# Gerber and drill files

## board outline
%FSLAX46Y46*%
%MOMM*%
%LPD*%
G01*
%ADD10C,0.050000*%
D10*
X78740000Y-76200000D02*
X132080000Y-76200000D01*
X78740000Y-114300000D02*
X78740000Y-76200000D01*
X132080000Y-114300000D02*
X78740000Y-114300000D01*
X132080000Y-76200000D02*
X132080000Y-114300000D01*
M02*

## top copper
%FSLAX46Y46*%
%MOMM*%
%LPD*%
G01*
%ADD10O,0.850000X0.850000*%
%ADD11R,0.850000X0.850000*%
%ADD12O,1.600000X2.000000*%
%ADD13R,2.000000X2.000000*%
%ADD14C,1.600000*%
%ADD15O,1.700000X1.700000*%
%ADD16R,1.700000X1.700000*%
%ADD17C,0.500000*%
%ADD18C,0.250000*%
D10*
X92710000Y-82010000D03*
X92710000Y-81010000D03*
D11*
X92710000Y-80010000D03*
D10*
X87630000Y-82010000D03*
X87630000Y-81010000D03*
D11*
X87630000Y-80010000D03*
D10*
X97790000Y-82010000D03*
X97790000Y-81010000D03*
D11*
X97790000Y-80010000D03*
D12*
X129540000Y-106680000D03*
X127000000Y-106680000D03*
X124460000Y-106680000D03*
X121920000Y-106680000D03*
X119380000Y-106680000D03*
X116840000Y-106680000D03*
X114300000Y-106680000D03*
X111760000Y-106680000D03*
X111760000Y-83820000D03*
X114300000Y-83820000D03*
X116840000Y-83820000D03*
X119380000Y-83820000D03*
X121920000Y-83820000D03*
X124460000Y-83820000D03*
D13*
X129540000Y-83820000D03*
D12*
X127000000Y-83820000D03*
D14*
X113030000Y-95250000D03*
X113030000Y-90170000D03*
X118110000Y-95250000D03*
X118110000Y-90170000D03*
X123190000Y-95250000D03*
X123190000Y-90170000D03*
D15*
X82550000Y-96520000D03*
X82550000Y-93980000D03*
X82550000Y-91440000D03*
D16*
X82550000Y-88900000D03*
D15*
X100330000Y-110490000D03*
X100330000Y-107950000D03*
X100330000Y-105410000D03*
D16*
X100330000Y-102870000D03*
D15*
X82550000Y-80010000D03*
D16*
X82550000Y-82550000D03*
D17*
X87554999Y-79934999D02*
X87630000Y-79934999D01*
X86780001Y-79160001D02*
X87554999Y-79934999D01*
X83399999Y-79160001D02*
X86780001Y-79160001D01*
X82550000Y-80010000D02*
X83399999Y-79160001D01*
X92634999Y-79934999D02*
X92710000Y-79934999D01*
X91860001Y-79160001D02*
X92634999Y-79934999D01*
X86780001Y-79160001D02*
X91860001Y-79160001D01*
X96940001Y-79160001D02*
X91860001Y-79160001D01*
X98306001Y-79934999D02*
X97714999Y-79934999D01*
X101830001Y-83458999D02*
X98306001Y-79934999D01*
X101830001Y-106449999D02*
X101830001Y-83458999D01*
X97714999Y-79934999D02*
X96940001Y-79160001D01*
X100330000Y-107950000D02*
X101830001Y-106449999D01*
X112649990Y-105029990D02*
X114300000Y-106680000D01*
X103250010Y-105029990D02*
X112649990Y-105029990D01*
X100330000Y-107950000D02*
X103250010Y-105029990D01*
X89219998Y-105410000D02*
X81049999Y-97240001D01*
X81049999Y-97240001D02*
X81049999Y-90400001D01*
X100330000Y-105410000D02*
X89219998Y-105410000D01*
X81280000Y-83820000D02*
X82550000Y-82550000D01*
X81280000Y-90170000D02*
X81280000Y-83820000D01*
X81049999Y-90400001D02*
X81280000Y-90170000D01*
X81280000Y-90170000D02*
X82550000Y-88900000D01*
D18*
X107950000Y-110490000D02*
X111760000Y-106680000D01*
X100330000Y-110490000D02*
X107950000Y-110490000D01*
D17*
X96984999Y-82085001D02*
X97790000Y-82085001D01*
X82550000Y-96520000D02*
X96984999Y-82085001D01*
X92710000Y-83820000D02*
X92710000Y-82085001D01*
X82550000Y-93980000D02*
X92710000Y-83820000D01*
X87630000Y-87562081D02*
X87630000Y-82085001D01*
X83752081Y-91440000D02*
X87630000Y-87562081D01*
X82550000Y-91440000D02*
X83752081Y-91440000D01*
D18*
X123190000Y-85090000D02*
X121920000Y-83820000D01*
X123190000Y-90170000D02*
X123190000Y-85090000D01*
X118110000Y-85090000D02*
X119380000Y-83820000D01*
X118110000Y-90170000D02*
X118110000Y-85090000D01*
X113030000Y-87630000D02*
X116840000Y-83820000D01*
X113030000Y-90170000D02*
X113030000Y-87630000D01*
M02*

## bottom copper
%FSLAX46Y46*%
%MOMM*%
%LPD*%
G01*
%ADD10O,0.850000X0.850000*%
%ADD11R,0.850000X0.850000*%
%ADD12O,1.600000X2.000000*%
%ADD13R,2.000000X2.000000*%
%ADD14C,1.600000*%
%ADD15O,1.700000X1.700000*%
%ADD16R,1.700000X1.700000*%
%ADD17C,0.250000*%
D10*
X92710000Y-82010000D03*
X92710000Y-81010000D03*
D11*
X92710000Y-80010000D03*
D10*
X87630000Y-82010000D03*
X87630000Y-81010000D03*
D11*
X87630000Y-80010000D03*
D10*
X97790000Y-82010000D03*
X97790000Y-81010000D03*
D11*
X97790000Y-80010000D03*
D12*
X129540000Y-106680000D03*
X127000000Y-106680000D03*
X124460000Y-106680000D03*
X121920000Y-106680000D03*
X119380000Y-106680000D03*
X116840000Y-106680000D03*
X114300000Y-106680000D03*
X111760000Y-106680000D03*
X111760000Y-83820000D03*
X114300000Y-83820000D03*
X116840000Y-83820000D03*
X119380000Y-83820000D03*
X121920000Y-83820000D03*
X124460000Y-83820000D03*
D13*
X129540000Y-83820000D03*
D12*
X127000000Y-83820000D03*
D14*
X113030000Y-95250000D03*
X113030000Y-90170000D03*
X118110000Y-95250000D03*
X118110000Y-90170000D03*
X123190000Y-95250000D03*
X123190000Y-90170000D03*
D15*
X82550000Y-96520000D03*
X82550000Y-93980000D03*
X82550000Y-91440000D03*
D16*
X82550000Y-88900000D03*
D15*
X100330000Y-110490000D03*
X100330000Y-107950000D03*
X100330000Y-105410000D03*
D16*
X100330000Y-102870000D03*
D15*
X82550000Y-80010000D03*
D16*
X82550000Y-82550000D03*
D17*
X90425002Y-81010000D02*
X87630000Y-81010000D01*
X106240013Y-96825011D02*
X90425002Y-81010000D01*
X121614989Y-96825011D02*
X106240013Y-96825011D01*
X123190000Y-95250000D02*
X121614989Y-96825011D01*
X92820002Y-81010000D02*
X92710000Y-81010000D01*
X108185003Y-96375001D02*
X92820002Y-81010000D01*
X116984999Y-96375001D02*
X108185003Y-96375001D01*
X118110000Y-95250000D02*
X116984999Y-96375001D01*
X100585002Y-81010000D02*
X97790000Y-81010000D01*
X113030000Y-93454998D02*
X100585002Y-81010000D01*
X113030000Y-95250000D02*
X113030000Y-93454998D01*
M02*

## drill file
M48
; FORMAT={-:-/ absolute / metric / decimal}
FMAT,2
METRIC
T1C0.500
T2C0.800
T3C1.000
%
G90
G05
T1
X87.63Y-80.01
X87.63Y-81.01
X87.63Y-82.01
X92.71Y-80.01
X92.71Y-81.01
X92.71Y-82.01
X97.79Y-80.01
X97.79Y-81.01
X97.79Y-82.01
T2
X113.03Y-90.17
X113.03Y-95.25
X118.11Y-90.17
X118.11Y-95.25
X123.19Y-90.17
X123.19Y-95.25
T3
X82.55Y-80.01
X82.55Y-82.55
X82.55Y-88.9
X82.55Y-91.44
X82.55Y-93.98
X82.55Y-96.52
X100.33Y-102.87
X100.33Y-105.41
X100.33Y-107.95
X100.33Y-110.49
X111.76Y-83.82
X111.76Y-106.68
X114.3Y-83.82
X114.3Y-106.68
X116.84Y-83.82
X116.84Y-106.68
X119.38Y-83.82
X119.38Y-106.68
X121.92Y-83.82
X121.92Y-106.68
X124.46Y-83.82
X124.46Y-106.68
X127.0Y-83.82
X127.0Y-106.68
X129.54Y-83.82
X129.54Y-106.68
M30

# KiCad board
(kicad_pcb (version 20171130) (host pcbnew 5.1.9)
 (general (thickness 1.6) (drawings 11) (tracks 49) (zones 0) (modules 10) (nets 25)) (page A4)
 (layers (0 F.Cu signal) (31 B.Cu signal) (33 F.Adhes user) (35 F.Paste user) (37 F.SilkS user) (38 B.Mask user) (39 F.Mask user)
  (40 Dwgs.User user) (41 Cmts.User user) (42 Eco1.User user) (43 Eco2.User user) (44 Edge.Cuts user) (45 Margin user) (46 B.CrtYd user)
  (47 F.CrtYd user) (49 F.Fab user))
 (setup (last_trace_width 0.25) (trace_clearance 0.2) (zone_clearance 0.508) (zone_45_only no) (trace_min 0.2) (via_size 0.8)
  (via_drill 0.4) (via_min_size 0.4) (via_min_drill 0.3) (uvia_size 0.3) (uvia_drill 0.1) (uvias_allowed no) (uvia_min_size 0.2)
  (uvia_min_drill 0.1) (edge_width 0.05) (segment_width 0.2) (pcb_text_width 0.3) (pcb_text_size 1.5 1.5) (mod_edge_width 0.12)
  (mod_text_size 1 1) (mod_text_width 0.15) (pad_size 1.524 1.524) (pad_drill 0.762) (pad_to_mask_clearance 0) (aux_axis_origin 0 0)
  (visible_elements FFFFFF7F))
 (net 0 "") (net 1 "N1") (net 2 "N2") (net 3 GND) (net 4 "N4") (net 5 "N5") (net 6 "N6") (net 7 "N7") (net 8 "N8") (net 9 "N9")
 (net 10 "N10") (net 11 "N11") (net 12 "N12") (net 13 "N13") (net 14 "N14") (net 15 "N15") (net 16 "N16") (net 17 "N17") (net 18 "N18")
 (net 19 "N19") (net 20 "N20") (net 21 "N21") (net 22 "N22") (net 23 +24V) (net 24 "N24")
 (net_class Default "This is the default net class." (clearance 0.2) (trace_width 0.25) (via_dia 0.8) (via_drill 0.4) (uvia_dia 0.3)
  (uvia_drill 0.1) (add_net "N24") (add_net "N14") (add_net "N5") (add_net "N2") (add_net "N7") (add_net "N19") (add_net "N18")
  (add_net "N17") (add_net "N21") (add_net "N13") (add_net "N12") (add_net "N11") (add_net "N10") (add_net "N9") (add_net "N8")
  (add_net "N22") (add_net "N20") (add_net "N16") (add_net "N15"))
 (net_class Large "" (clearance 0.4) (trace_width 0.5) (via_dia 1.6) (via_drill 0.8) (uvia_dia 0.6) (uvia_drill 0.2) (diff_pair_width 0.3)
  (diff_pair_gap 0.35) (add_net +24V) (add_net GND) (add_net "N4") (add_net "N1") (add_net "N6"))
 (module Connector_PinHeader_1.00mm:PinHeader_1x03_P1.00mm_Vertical (layer F.Cu) (at 92.71 80.01)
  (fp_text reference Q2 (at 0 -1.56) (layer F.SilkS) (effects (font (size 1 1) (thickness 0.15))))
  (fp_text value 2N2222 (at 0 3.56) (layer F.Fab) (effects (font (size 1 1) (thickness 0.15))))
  (pad 3 thru_hole oval (at 0 2) (size 0.85 0.85) (drill 0.5) (layers *.Cu *.Mask) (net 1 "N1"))
  (pad 2 thru_hole oval (at 0 1) (size 0.85 0.85) (drill 0.5) (layers *.Cu *.Mask) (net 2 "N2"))
  (pad 1 thru_hole rect (at 0 0) (size 0.85 0.85) (drill 0.5) (layers *.Cu *.Mask) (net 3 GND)))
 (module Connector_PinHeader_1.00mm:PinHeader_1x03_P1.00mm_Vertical (layer F.Cu) (at 87.63 80.01)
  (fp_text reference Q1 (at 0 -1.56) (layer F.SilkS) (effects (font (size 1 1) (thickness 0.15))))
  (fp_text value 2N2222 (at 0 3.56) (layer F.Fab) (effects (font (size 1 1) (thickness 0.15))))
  (pad 3 thru_hole oval (at 0 2) (size 0.85 0.85) (drill 0.5) (layers *.Cu *.Mask) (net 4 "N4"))
  (pad 2 thru_hole oval (at 0 1) (size 0.85 0.85) (drill 0.5) (layers *.Cu *.Mask) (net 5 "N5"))
  (pad 1 thru_hole rect (at 0 0) (size 0.85 0.85) (drill 0.5) (layers *.Cu *.Mask) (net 3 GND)))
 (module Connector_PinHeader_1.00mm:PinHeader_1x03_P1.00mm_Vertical (layer F.Cu) (at 97.79 80.01)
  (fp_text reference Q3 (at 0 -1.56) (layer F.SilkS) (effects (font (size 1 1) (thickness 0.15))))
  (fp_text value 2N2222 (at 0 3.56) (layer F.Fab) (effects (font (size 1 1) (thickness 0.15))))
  (pad 3 thru_hole oval (at 0 2) (size 0.85 0.85) (drill 0.5) (layers *.Cu *.Mask) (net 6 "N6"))
  (pad 2 thru_hole oval (at 0 1) (size 0.85 0.85) (drill 0.5) (layers *.Cu *.Mask) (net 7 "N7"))
  (pad 1 thru_hole rect (at 0 0) (size 0.85 0.85) (drill 0.5) (layers *.Cu *.Mask) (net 3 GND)))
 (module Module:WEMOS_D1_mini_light (layer F.Cu) (at 129.54 83.82 270)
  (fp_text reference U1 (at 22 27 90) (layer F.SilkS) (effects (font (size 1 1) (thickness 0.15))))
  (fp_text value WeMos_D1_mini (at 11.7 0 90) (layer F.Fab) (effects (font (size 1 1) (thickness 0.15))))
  (pad 16 thru_hole oval (at 22.86 0 270) (size 2 1.6) (drill 1) (layers *.Cu *.Mask) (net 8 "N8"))
  (pad 15 thru_hole oval (at 22.86 2.54 270) (size 2 1.6) (drill 1) (layers *.Cu *.Mask) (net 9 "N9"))
  (pad 14 thru_hole oval (at 22.86 5.08 270) (size 2 1.6) (drill 1) (layers *.Cu *.Mask) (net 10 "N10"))
  (pad 13 thru_hole oval (at 22.86 7.62 270) (size 2 1.6) (drill 1) (layers *.Cu *.Mask) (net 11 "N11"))
  (pad 12 thru_hole oval (at 22.86 10.16 270) (size 2 1.6) (drill 1) (layers *.Cu *.Mask) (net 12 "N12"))
  (pad 11 thru_hole oval (at 22.86 12.7 270) (size 2 1.6) (drill 1) (layers *.Cu *.Mask) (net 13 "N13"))
  (pad 10 thru_hole oval (at 22.86 15.24 270) (size 2 1.6) (drill 1) (layers *.Cu *.Mask) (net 3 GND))
  (pad 9 thru_hole oval (at 22.86 17.78 270) (size 2 1.6) (drill 1) (layers *.Cu *.Mask) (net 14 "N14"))
  (pad 8 thru_hole oval (at 0 17.78 270) (size 2 1.6) (drill 1) (layers *.Cu *.Mask) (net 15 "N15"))
  (pad 7 thru_hole oval (at 0 15.24 270) (size 2 1.6) (drill 1) (layers *.Cu *.Mask) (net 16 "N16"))
  (pad 6 thru_hole oval (at 0 12.7 270) (size 2 1.6) (drill 1) (layers *.Cu *.Mask) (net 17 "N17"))
  (pad 5 thru_hole oval (at 0 10.16 270) (size 2 1.6) (drill 1) (layers *.Cu *.Mask) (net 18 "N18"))
  (pad 4 thru_hole oval (at 0 7.62 270) (size 2 1.6) (drill 1) (layers *.Cu *.Mask) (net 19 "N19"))
  (pad 3 thru_hole oval (at 0 5.08 270) (size 2 1.6) (drill 1) (layers *.Cu *.Mask) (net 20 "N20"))
  (pad 1 thru_hole rect (at 0 0 270) (size 2 2) (drill 1) (layers *.Cu *.Mask) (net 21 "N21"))
  (pad 2 thru_hole oval (at 0 2.54 270) (size 2 1.6) (drill 1) (layers *.Cu *.Mask) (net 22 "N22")))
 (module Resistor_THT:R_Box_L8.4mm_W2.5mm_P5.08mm (layer F.Cu) (at 113.03 90.17 270)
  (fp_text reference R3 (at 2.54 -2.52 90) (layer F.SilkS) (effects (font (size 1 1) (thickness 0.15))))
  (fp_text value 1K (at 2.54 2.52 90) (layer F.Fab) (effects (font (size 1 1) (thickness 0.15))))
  (pad 2 thru_hole circle (at 5.08 0 270) (size 1.6 1.6) (drill 0.8) (layers *.Cu *.Mask) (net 7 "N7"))
  (pad 1 thru_hole circle (at 0 0 270) (size 1.6 1.6) (drill 0.8) (layers *.Cu *.Mask) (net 17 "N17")))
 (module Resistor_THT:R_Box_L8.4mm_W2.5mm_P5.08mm (layer F.Cu) (at 118.11 90.17 270)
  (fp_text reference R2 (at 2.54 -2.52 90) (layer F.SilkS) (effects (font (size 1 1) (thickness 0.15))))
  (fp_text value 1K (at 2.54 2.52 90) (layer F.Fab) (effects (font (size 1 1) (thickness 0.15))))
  (pad 2 thru_hole circle (at 5.08 0 270) (size 1.6 1.6) (drill 0.8) (layers *.Cu *.Mask) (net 2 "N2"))
  (pad 1 thru_hole circle (at 0 0 270) (size 1.6 1.6) (drill 0.8) (layers *.Cu *.Mask) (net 18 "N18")))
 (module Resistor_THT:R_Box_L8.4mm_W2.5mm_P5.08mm (layer F.Cu) (at 123.19 90.17 270)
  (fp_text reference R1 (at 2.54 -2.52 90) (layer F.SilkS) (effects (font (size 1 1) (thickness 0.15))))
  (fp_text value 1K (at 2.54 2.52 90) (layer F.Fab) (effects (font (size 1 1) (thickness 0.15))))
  (pad 2 thru_hole circle (at 5.08 0 270) (size 1.6 1.6) (drill 0.8) (layers *.Cu *.Mask) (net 5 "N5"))
  (pad 1 thru_hole circle (at 0 0 270) (size 1.6 1.6) (drill 0.8) (layers *.Cu *.Mask) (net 19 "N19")))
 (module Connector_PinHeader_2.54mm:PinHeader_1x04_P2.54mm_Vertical (layer F.Cu) (at 82.55 88.9)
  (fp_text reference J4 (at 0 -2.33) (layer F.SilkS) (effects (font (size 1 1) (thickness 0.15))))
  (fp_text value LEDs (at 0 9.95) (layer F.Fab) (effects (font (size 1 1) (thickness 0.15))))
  (pad 4 thru_hole oval (at 0 7.62) (size 1.7 1.7) (drill 1) (layers *.Cu *.Mask) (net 6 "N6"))
  (pad 3 thru_hole oval (at 0 5.08) (size 1.7 1.7) (drill 1) (layers *.Cu *.Mask) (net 1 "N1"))
  (pad 2 thru_hole oval (at 0 2.54) (size 1.7 1.7) (drill 1) (layers *.Cu *.Mask) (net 4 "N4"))
  (pad 1 thru_hole rect (at 0 0) (size 1.7 1.7) (drill 1) (layers *.Cu *.Mask) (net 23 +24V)))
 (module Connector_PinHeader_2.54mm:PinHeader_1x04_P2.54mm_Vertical (layer F.Cu) (at 100.33 102.87)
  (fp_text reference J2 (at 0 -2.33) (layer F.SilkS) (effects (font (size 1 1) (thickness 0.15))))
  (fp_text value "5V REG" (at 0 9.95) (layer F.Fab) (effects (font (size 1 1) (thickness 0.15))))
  (pad 4 thru_hole oval (at 0 7.62) (size 1.7 1.7) (drill 1) (layers *.Cu *.Mask) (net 14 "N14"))
  (pad 3 thru_hole oval (at 0 5.08) (size 1.7 1.7) (drill 1) (layers *.Cu *.Mask) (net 3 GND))
  (pad 2 thru_hole oval (at 0 2.54) (size 1.7 1.7) (drill 1) (layers *.Cu *.Mask) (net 23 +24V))
  (pad 1 thru_hole rect (at 0 0) (size 1.7 1.7) (drill 1) (layers *.Cu *.Mask) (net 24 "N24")))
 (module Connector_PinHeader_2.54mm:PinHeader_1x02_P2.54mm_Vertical (layer F.Cu) (at 82.55 82.55 180)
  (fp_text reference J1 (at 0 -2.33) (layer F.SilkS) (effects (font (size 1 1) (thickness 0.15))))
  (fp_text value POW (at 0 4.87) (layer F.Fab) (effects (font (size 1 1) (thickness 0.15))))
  (pad 2 thru_hole oval (at 0 2.54 180) (size 1.7 1.7) (drill 1) (layers *.Cu *.Mask) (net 3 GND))
  (pad 1 thru_hole rect (at 0 0 180) (size 1.7 1.7) (drill 1) (layers *.Cu *.Mask) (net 23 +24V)))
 (gr_line (start 78.74 76.2) (end 132.08 76.2) (layer Edge.Cuts) (width 0.05))
 (gr_line (start 78.74 114.3) (end 78.74 76.2) (layer Edge.Cuts) (width 0.05))
 (gr_line (start 132.08 114.3) (end 78.74 114.3) (layer Edge.Cuts) (width 0.05))
 (gr_line (start 132.08 76.2) (end 132.08 114.3) (layer Edge.Cuts) (width 0.05))
 (segment (start 87.554999 79.934999) (end 87.63 79.934999) (width 0.5) (layer F.Cu) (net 3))
 (segment (start 86.780001 79.160001) (end 87.554999 79.934999) (width 0.5) (layer F.Cu) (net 3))
 (segment (start 83.399999 79.160001) (end 86.780001 79.160001) (width 0.5) (layer F.Cu) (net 3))
 (segment (start 82.55 80.01) (end 83.399999 79.160001) (width 0.5) (layer F.Cu) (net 3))
 (segment (start 92.634999 79.934999) (end 92.71 79.934999) (width 0.5) (layer F.Cu) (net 3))
 (segment (start 91.860001 79.160001) (end 92.634999 79.934999) (width 0.5) (layer F.Cu) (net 3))
 (segment (start 86.780001 79.160001) (end 91.860001 79.160001) (width 0.5) (layer F.Cu) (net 3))
 (segment (start 96.940001 79.160001) (end 91.860001 79.160001) (width 0.5) (layer F.Cu) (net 3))
 (segment (start 98.306001 79.934999) (end 97.714999 79.934999) (width 0.5) (layer F.Cu) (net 3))
 (segment (start 101.830001 83.458999) (end 98.306001 79.934999) (width 0.5) (layer F.Cu) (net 3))
 (segment (start 101.830001 106.449999) (end 101.830001 83.458999) (width 0.5) (layer F.Cu) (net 3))
 (segment (start 97.714999 79.934999) (end 96.940001 79.160001) (width 0.5) (layer F.Cu) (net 3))
 (segment (start 100.33 107.95) (end 101.830001 106.449999) (width 0.5) (layer F.Cu) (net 3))
 (segment (start 112.64999 105.02999) (end 114.3 106.68) (width 0.5) (layer F.Cu) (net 3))
 (segment (start 103.25001 105.02999) (end 112.64999 105.02999) (width 0.5) (layer F.Cu) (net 3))
 (segment (start 100.33 107.95) (end 103.25001 105.02999) (width 0.5) (layer F.Cu) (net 3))
 (segment (start 89.219998 105.41) (end 81.049999 97.240001) (width 0.5) (layer F.Cu) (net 23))
 (segment (start 81.049999 97.240001) (end 81.049999 90.400001) (width 0.5) (layer F.Cu) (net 23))
 (segment (start 100.33 105.41) (end 89.219998 105.41) (width 0.5) (layer F.Cu) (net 23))
 (segment (start 81.28 83.82) (end 82.55 82.55) (width 0.5) (layer F.Cu) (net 23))
 (segment (start 81.28 90.17) (end 81.28 83.82) (width 0.5) (layer F.Cu) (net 23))
 (segment (start 81.049999 90.400001) (end 81.28 90.17) (width 0.5) (layer F.Cu) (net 23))
 (segment (start 81.28 90.17) (end 82.55 88.9) (width 0.5) (layer F.Cu) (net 23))
 (segment (start 107.95 110.49) (end 111.76 106.68) (width 0.25) (layer F.Cu) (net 14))
 (segment (start 100.33 110.49) (end 107.95 110.49) (width 0.25) (layer F.Cu) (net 14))
 (segment (start 96.984999 82.085001) (end 97.79 82.085001) (width 0.5) (layer F.Cu) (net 6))
 (segment (start 82.55 96.52) (end 96.984999 82.085001) (width 0.5) (layer F.Cu) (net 6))
 (segment (start 92.71 83.82) (end 92.71 82.085001) (width 0.5) (layer F.Cu) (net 1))
 (segment (start 82.55 93.98) (end 92.71 83.82) (width 0.5) (layer F.Cu) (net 1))
 (segment (start 87.63 87.562081) (end 87.63 82.085001) (width 0.5) (layer F.Cu) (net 4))
 (segment (start 83.752081 91.44) (end 87.63 87.562081) (width 0.5) (layer F.Cu) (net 4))
 (segment (start 82.55 91.44) (end 83.752081 91.44) (width 0.5) (layer F.Cu) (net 4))
 (segment (start 90.425002 81.01) (end 87.63 81.01) (width 0.25) (layer B.Cu) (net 5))
 (segment (start 106.240013 96.825011) (end 90.425002 81.01) (width 0.25) (layer B.Cu) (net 5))
 (segment (start 121.614989 96.825011) (end 106.240013 96.825011) (width 0.25) (layer B.Cu) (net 5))
 (segment (start 123.19 95.25) (end 121.614989 96.825011) (width 0.25) (layer B.Cu) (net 5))
 (segment (start 92.820002 81.01) (end 92.71 81.01) (width 0.25) (layer B.Cu) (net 2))
 (segment (start 108.185003 96.375001) (end 92.820002 81.01) (width 0.25) (layer B.Cu) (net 2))
 (segment (start 116.984999 96.375001) (end 108.185003 96.375001) (width 0.25) (layer B.Cu) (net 2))
 (segment (start 118.11 95.25) (end 116.984999 96.375001) (width 0.25) (layer B.Cu) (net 2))
 (segment (start 100.585002 81.01) (end 97.79 81.01) (width 0.25) (layer B.Cu) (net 7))
 (segment (start 113.03 93.454998) (end 100.585002 81.01) (width 0.25) (layer B.Cu) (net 7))
 (segment (start 113.03 95.25) (end 113.03 93.454998) (width 0.25) (layer B.Cu) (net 7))
 (segment (start 123.19 85.09) (end 121.92 83.82) (width 0.25) (layer F.Cu) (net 19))
 (segment (start 123.19 90.17) (end 123.19 85.09) (width 0.25) (layer F.Cu) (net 19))
 (segment (start 118.11 85.09) (end 119.38 83.82) (width 0.25) (layer F.Cu) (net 18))
 (segment (start 118.11 90.17) (end 118.11 85.09) (width 0.25) (layer F.Cu) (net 18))
 (segment (start 113.03 87.63) (end 116.84 83.82) (width 0.25) (layer F.Cu) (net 17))
 (segment (start 113.03 90.17) (end 113.03 87.63) (width 0.25) (layer F.Cu) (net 17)))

